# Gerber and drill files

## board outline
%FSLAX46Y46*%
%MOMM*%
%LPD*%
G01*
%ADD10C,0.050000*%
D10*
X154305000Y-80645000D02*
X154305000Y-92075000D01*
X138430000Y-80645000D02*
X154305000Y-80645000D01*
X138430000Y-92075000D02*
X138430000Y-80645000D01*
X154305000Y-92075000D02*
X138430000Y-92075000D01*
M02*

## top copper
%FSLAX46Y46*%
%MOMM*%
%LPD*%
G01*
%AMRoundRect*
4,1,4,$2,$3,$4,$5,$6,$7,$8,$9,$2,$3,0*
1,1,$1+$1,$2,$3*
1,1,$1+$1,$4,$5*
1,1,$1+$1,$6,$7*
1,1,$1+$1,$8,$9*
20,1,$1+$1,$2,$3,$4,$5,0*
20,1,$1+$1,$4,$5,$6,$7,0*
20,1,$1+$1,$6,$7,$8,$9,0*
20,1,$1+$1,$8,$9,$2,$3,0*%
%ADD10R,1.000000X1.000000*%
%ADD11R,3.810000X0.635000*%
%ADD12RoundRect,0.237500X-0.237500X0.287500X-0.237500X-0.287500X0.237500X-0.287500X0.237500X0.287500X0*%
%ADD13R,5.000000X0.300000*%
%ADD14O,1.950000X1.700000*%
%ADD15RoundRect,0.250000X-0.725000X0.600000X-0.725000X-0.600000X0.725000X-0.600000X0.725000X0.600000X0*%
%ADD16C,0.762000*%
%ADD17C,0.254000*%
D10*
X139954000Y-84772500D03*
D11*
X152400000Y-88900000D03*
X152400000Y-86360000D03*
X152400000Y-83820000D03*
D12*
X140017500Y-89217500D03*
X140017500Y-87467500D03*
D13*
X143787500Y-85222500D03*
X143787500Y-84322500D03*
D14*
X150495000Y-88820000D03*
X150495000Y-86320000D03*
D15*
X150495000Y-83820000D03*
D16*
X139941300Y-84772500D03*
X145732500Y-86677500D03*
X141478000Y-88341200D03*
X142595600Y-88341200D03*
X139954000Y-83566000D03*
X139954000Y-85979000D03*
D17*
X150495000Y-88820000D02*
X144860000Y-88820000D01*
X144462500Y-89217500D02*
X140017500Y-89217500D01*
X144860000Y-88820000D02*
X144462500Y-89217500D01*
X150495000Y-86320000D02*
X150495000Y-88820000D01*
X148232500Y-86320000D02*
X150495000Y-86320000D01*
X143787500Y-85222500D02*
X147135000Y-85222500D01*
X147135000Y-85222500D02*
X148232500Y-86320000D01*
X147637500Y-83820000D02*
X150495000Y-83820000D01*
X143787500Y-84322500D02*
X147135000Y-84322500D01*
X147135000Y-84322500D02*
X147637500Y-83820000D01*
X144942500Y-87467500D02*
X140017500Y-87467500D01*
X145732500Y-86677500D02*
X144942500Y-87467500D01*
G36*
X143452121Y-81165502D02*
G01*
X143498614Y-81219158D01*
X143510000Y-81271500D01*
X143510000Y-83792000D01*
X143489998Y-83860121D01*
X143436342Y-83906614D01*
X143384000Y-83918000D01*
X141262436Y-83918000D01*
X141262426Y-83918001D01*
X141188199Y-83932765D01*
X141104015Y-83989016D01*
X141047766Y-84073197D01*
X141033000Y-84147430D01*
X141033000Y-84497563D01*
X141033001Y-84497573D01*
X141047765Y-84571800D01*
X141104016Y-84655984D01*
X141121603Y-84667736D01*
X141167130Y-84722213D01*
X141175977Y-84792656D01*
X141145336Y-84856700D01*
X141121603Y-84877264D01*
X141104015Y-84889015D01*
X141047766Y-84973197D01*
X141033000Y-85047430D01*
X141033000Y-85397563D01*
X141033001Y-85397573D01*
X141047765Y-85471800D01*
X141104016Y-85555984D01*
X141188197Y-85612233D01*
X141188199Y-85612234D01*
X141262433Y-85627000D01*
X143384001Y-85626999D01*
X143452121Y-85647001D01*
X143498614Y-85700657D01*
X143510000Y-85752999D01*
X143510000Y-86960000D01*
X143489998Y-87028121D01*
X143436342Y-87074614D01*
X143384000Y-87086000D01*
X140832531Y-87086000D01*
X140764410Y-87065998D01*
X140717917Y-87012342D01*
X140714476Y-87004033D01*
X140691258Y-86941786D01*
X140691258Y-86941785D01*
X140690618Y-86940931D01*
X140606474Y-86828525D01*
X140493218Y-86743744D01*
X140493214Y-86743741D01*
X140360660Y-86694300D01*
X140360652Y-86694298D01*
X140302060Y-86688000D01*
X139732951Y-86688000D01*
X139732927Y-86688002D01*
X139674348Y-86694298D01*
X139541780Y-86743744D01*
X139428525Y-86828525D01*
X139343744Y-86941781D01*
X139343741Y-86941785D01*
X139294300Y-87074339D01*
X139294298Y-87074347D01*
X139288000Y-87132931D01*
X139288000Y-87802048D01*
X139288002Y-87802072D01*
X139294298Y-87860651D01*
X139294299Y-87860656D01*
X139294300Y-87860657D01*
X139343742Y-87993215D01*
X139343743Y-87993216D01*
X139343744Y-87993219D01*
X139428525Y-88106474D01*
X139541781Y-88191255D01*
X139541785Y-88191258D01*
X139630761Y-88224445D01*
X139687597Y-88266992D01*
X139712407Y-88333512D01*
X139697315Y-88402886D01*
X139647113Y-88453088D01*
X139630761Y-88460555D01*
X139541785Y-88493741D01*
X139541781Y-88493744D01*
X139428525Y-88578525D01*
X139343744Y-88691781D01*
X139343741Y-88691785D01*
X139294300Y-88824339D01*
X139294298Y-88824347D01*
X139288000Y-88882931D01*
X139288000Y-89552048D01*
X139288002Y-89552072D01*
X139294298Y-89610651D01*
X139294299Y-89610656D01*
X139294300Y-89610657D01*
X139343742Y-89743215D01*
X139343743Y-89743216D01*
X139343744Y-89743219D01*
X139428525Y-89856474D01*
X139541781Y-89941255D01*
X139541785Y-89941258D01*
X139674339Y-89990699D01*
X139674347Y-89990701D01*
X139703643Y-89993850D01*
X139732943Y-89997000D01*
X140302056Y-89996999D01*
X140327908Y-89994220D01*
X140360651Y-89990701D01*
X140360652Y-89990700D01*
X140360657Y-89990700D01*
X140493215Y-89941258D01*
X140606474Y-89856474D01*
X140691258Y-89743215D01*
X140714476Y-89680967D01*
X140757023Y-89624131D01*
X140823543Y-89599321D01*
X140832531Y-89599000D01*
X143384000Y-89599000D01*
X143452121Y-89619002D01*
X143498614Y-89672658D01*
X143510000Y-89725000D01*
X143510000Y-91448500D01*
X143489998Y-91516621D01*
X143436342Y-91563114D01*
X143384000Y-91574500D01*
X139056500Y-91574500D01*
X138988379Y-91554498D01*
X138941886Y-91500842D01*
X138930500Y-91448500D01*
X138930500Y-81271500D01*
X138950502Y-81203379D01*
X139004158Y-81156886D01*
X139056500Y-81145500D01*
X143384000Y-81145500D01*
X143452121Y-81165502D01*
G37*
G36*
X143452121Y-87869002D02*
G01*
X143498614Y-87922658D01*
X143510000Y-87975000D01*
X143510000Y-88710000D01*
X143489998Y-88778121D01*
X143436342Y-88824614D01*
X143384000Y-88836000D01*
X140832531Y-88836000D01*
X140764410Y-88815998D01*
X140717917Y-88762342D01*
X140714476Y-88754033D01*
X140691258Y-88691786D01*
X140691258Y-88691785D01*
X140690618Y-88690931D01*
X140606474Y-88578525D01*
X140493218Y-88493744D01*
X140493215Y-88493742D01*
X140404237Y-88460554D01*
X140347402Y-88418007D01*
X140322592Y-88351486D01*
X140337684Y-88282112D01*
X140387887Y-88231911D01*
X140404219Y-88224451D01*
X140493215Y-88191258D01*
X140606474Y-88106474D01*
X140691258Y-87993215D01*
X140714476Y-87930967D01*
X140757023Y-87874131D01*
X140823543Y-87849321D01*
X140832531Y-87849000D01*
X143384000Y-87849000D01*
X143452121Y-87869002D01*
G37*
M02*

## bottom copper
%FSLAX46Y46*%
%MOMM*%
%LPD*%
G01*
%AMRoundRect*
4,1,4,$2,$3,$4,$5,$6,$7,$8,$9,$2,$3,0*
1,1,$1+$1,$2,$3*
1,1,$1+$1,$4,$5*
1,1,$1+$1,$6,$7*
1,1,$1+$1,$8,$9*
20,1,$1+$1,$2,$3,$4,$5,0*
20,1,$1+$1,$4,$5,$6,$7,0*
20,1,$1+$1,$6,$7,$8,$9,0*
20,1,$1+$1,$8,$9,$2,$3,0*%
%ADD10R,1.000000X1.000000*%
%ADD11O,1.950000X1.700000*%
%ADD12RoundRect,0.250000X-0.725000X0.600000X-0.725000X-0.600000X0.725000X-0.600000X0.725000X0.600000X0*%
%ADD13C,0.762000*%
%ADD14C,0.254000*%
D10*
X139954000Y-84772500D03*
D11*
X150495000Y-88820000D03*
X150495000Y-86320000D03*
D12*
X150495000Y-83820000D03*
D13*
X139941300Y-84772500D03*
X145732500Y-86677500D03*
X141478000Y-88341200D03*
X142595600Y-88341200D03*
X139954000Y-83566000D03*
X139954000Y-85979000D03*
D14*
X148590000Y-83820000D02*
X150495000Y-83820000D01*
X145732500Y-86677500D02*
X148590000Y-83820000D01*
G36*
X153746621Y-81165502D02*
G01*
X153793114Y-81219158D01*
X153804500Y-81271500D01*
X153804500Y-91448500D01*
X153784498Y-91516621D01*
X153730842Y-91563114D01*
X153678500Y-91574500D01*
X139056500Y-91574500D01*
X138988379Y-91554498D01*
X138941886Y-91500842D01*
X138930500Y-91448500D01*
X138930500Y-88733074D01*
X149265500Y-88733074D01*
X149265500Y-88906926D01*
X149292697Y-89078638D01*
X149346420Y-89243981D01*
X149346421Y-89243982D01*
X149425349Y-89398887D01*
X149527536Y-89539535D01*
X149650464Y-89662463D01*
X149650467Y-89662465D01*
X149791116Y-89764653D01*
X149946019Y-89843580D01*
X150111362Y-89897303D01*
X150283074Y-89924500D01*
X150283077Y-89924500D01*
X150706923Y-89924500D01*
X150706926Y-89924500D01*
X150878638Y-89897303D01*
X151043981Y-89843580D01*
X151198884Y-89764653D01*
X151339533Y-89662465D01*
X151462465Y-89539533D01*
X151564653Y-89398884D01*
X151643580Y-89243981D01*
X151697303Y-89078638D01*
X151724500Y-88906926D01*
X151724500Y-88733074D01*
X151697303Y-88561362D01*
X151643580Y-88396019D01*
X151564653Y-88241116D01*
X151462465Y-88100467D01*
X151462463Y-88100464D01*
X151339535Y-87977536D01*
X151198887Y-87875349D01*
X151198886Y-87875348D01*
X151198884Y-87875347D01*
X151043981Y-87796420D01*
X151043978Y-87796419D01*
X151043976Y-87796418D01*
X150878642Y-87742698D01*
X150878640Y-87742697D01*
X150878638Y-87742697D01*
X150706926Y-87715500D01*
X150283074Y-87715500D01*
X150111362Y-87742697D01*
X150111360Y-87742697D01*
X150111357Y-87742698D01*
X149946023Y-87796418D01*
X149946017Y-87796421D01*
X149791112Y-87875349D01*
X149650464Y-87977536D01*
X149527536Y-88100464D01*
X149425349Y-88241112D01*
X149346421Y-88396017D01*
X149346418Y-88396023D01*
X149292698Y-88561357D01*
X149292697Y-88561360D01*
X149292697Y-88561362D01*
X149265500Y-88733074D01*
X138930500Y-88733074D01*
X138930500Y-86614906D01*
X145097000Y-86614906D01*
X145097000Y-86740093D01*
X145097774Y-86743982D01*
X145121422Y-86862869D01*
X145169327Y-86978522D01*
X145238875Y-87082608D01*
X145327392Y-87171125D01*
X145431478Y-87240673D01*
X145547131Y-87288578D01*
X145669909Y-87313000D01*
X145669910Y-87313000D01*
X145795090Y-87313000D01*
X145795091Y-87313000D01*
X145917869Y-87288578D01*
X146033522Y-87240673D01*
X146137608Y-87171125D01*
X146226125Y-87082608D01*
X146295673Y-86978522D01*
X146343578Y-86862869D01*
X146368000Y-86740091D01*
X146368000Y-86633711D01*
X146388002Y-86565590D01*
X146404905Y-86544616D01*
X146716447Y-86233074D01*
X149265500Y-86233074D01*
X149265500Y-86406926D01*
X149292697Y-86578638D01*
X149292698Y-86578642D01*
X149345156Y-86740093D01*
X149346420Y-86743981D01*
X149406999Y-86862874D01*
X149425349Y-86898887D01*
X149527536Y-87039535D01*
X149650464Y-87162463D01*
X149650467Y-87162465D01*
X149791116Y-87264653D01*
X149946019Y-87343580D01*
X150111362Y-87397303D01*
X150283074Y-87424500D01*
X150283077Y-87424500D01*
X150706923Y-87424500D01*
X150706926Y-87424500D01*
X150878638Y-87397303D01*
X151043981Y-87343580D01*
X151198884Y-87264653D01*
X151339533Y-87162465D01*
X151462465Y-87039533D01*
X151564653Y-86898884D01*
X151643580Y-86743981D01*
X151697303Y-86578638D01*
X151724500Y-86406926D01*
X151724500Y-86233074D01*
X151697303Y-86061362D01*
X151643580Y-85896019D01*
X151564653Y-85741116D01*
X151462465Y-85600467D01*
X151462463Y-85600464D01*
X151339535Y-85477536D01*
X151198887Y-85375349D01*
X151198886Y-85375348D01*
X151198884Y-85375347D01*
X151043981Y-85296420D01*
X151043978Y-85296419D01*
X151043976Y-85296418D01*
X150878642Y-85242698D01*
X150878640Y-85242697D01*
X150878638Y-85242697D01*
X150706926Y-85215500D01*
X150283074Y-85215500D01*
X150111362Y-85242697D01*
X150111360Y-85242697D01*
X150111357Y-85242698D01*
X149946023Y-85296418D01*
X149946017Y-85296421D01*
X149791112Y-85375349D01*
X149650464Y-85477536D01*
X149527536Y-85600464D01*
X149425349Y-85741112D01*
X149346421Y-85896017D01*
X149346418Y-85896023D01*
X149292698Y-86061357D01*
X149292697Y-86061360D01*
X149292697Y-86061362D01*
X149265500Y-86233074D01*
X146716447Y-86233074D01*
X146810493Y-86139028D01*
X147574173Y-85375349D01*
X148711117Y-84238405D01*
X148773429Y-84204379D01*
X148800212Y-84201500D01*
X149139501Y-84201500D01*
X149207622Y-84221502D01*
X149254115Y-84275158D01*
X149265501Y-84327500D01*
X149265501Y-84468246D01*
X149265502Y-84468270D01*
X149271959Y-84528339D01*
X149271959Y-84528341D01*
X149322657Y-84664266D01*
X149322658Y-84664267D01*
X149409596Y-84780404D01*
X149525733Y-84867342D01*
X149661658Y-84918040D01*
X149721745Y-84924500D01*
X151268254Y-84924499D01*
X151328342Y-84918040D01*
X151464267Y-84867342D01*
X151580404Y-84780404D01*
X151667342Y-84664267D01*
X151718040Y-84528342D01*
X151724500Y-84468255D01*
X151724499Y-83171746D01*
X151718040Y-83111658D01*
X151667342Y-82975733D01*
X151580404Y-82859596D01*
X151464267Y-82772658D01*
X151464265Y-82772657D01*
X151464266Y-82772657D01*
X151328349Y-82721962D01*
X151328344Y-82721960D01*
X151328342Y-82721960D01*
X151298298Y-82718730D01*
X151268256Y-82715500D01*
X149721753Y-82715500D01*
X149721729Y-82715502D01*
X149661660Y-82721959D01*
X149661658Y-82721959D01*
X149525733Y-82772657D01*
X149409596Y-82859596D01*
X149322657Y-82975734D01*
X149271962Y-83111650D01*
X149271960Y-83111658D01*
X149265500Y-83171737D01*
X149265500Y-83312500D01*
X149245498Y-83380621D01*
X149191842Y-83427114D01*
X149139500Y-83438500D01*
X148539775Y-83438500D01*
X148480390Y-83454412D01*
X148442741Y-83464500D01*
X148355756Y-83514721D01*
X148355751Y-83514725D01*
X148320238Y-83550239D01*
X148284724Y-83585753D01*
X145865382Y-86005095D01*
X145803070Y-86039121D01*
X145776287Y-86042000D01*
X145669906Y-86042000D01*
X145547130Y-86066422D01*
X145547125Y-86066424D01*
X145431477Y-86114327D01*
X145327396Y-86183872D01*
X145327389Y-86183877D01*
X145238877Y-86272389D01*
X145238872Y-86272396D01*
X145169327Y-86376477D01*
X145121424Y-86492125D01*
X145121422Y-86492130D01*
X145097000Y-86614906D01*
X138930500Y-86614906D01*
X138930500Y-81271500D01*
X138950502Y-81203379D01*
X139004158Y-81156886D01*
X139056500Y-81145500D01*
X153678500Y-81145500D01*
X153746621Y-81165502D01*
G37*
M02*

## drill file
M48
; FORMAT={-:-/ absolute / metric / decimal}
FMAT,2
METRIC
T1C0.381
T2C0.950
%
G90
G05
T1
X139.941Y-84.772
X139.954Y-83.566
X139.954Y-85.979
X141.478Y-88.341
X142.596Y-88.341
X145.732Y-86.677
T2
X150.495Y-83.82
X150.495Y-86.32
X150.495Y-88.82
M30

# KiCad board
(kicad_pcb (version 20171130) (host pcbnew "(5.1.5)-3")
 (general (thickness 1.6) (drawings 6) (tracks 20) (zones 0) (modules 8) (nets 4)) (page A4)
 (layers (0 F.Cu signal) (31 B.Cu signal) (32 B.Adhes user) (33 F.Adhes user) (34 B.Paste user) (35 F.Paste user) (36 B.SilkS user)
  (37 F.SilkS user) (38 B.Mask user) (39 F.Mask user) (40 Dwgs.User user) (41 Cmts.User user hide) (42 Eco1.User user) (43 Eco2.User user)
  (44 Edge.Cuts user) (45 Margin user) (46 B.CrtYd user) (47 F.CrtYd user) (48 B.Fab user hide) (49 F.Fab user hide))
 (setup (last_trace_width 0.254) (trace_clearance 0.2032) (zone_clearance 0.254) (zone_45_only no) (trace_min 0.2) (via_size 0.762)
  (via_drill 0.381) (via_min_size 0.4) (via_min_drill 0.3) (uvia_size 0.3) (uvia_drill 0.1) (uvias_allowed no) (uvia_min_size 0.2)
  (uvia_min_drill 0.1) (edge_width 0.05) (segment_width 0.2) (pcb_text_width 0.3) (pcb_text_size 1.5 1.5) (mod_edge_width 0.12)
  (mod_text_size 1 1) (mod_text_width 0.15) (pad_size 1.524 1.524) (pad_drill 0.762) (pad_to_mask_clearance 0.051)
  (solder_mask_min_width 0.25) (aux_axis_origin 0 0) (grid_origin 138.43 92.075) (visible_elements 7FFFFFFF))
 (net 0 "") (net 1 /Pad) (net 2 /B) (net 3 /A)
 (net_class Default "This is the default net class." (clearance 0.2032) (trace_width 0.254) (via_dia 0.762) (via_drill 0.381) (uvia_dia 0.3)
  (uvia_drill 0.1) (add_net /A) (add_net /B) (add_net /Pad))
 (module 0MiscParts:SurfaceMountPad (layer F.Cu) (at 139.954 84.7725)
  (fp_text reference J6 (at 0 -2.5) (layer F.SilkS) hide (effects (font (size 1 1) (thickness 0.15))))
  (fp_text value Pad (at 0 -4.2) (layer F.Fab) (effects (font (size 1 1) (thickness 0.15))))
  (pad 1 smd rect (at 0 0) (size 1 1) (layers F.Cu F.Paste F.Mask) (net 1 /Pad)))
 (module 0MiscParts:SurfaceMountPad (layer B.Cu) (at 139.954 84.7725)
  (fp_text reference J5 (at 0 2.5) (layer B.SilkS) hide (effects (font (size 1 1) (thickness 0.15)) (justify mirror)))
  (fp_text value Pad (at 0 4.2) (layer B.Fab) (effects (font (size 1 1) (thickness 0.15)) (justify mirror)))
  (pad 1 smd rect (at 0 0) (size 1 1) (layers B.Cu B.Paste B.Mask) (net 1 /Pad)))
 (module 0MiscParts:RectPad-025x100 (layer F.Cu) (at 150.495 88.9)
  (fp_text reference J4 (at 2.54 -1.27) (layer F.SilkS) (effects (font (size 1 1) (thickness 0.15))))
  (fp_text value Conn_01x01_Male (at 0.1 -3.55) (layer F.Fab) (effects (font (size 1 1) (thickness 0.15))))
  (pad 1 smd rect (at 1.905 0) (size 3.81 0.635) (layers F.Cu F.Paste F.Mask) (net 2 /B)))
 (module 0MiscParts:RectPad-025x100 (layer F.Cu) (at 150.495 86.36)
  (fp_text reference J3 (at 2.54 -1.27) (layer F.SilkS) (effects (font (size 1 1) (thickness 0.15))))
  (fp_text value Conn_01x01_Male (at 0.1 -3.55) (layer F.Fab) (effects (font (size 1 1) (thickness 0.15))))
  (pad 1 smd rect (at 1.905 0) (size 3.81 0.635) (layers F.Cu F.Paste F.Mask) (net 2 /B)))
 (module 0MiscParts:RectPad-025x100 (layer F.Cu) (at 150.495 83.82)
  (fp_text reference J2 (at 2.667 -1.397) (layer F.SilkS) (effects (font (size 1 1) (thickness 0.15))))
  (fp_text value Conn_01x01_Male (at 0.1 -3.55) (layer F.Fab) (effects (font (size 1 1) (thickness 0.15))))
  (pad 1 smd rect (at 1.905 0) (size 3.81 0.635) (layers F.Cu F.Paste F.Mask) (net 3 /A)))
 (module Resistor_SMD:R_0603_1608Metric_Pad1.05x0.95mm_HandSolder (layer F.Cu) (at 140.0175 88.3425 270)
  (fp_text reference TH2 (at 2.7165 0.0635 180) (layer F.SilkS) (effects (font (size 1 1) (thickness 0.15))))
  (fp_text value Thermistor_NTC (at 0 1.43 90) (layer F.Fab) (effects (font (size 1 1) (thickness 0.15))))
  (pad 2 smd roundrect (at 0.875 0 270) (size 1.05 0.95) (layers F.Cu F.Paste F.Mask) (roundrect_rratio 0.25) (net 2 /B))
  (pad 1 smd roundrect (at -0.875 0 270) (size 1.05 0.95) (layers F.Cu F.Paste F.Mask) (roundrect_rratio 0.25) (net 3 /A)))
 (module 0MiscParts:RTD (layer F.Cu) (at 141.2875 84.7725)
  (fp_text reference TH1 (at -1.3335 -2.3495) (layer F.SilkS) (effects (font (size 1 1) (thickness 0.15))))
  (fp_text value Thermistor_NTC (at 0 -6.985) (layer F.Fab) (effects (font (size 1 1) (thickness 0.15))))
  (pad 2 smd rect (at 2.5 0.45) (size 5 0.3) (layers F.Cu F.Paste F.Mask) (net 2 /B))
  (pad 1 smd rect (at 2.5 -0.45) (size 5 0.3) (layers F.Cu F.Paste F.Mask) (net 3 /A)))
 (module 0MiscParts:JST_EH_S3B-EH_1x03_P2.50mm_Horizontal (layer F.Cu) (at 150.495 83.82 270)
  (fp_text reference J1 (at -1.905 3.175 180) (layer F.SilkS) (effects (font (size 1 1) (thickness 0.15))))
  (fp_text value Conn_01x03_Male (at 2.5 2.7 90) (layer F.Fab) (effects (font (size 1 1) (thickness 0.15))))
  (pad 3 thru_hole oval (at 5 0 270) (size 1.7 1.95) (drill 0.95) (layers *.Cu *.Mask) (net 2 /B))
  (pad 2 thru_hole oval (at 2.5 0 270) (size 1.7 1.95) (drill 0.95) (layers *.Cu *.Mask) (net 2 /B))
  (pad 1 thru_hole roundrect (at 0 0 270) (size 1.7 1.95) (drill 0.95) (layers *.Cu *.Mask) (roundrect_rratio 0.147059) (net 3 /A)))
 (gr_line (start 154.305 80.645) (end 154.305 92.075) (layer Edge.Cuts) (width 0.05))
 (gr_line (start 138.43 80.645) (end 154.305 80.645) (layer Edge.Cuts) (width 0.05))
 (gr_line (start 138.43 92.075) (end 138.43 80.645) (layer Edge.Cuts) (width 0.05))
 (gr_line (start 154.305 92.075) (end 138.43 92.075) (layer Edge.Cuts) (width 0.05))
 (via (at 139.9413 84.7725) (size 0.762) (drill 0.381) (layers F.Cu B.Cu) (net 1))
 (segment (start 150.495 88.82) (end 144.86 88.82) (width 0.254) (layer F.Cu) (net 2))
 (segment (start 144.4625 89.2175) (end 140.0175 89.2175) (width 0.254) (layer F.Cu) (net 2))
 (segment (start 144.86 88.82) (end 144.4625 89.2175) (width 0.254) (layer F.Cu) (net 2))
 (segment (start 150.495 86.32) (end 150.495 88.82) (width 0.254) (layer F.Cu) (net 2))
 (segment (start 148.2325 86.32) (end 150.495 86.32) (width 0.254) (layer F.Cu) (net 2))
 (segment (start 143.7875 85.2225) (end 147.135 85.2225) (width 0.254) (layer F.Cu) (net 2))
 (segment (start 147.135 85.2225) (end 148.2325 86.32) (width 0.254) (layer F.Cu) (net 2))
 (segment (start 147.6375 83.82) (end 150.495 83.82) (width 0.254) (layer F.Cu) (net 3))
 (segment (start 143.7875 84.3225) (end 147.135 84.3225) (width 0.254) (layer F.Cu) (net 3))
 (segment (start 147.135 84.3225) (end 147.6375 83.82) (width 0.254) (layer F.Cu) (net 3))
 (segment (start 148.59 83.82) (end 150.495 83.82) (width 0.254) (layer B.Cu) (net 3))
 (segment (start 144.9425 87.4675) (end 140.0175 87.4675) (width 0.254) (layer F.Cu) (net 3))
 (segment (start 145.7325 86.6775) (end 148.59 83.82) (width 0.254) (layer B.Cu) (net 3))
 (via (at 145.7325 86.6775) (size 0.762) (drill 0.381) (layers F.Cu B.Cu) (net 3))
 (segment (start 145.7325 86.6775) (end 144.9425 87.4675) (width 0.254) (layer F.Cu) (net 3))
 (via (at 141.478 88.3412) (size 0.762) (drill 0.381) (layers F.Cu B.Cu) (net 1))
 (via (at 142.5956 88.3412) (size 0.762) (drill 0.381) (layers F.Cu B.Cu) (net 1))
 (via (at 139.954 83.566) (size 0.762) (drill 0.381) (layers F.Cu B.Cu) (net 1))
 (via (at 139.954 85.979) (size 0.762) (drill 0.381) (layers F.Cu B.Cu) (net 1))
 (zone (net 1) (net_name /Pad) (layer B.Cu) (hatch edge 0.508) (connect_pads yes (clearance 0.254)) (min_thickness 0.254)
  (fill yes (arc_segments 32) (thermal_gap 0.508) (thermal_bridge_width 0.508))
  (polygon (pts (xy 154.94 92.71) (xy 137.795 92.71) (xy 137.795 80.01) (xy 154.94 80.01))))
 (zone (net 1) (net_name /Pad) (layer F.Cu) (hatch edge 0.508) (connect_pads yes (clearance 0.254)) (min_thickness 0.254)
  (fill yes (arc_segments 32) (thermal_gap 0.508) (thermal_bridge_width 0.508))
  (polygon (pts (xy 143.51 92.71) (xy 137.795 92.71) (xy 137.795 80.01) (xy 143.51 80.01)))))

